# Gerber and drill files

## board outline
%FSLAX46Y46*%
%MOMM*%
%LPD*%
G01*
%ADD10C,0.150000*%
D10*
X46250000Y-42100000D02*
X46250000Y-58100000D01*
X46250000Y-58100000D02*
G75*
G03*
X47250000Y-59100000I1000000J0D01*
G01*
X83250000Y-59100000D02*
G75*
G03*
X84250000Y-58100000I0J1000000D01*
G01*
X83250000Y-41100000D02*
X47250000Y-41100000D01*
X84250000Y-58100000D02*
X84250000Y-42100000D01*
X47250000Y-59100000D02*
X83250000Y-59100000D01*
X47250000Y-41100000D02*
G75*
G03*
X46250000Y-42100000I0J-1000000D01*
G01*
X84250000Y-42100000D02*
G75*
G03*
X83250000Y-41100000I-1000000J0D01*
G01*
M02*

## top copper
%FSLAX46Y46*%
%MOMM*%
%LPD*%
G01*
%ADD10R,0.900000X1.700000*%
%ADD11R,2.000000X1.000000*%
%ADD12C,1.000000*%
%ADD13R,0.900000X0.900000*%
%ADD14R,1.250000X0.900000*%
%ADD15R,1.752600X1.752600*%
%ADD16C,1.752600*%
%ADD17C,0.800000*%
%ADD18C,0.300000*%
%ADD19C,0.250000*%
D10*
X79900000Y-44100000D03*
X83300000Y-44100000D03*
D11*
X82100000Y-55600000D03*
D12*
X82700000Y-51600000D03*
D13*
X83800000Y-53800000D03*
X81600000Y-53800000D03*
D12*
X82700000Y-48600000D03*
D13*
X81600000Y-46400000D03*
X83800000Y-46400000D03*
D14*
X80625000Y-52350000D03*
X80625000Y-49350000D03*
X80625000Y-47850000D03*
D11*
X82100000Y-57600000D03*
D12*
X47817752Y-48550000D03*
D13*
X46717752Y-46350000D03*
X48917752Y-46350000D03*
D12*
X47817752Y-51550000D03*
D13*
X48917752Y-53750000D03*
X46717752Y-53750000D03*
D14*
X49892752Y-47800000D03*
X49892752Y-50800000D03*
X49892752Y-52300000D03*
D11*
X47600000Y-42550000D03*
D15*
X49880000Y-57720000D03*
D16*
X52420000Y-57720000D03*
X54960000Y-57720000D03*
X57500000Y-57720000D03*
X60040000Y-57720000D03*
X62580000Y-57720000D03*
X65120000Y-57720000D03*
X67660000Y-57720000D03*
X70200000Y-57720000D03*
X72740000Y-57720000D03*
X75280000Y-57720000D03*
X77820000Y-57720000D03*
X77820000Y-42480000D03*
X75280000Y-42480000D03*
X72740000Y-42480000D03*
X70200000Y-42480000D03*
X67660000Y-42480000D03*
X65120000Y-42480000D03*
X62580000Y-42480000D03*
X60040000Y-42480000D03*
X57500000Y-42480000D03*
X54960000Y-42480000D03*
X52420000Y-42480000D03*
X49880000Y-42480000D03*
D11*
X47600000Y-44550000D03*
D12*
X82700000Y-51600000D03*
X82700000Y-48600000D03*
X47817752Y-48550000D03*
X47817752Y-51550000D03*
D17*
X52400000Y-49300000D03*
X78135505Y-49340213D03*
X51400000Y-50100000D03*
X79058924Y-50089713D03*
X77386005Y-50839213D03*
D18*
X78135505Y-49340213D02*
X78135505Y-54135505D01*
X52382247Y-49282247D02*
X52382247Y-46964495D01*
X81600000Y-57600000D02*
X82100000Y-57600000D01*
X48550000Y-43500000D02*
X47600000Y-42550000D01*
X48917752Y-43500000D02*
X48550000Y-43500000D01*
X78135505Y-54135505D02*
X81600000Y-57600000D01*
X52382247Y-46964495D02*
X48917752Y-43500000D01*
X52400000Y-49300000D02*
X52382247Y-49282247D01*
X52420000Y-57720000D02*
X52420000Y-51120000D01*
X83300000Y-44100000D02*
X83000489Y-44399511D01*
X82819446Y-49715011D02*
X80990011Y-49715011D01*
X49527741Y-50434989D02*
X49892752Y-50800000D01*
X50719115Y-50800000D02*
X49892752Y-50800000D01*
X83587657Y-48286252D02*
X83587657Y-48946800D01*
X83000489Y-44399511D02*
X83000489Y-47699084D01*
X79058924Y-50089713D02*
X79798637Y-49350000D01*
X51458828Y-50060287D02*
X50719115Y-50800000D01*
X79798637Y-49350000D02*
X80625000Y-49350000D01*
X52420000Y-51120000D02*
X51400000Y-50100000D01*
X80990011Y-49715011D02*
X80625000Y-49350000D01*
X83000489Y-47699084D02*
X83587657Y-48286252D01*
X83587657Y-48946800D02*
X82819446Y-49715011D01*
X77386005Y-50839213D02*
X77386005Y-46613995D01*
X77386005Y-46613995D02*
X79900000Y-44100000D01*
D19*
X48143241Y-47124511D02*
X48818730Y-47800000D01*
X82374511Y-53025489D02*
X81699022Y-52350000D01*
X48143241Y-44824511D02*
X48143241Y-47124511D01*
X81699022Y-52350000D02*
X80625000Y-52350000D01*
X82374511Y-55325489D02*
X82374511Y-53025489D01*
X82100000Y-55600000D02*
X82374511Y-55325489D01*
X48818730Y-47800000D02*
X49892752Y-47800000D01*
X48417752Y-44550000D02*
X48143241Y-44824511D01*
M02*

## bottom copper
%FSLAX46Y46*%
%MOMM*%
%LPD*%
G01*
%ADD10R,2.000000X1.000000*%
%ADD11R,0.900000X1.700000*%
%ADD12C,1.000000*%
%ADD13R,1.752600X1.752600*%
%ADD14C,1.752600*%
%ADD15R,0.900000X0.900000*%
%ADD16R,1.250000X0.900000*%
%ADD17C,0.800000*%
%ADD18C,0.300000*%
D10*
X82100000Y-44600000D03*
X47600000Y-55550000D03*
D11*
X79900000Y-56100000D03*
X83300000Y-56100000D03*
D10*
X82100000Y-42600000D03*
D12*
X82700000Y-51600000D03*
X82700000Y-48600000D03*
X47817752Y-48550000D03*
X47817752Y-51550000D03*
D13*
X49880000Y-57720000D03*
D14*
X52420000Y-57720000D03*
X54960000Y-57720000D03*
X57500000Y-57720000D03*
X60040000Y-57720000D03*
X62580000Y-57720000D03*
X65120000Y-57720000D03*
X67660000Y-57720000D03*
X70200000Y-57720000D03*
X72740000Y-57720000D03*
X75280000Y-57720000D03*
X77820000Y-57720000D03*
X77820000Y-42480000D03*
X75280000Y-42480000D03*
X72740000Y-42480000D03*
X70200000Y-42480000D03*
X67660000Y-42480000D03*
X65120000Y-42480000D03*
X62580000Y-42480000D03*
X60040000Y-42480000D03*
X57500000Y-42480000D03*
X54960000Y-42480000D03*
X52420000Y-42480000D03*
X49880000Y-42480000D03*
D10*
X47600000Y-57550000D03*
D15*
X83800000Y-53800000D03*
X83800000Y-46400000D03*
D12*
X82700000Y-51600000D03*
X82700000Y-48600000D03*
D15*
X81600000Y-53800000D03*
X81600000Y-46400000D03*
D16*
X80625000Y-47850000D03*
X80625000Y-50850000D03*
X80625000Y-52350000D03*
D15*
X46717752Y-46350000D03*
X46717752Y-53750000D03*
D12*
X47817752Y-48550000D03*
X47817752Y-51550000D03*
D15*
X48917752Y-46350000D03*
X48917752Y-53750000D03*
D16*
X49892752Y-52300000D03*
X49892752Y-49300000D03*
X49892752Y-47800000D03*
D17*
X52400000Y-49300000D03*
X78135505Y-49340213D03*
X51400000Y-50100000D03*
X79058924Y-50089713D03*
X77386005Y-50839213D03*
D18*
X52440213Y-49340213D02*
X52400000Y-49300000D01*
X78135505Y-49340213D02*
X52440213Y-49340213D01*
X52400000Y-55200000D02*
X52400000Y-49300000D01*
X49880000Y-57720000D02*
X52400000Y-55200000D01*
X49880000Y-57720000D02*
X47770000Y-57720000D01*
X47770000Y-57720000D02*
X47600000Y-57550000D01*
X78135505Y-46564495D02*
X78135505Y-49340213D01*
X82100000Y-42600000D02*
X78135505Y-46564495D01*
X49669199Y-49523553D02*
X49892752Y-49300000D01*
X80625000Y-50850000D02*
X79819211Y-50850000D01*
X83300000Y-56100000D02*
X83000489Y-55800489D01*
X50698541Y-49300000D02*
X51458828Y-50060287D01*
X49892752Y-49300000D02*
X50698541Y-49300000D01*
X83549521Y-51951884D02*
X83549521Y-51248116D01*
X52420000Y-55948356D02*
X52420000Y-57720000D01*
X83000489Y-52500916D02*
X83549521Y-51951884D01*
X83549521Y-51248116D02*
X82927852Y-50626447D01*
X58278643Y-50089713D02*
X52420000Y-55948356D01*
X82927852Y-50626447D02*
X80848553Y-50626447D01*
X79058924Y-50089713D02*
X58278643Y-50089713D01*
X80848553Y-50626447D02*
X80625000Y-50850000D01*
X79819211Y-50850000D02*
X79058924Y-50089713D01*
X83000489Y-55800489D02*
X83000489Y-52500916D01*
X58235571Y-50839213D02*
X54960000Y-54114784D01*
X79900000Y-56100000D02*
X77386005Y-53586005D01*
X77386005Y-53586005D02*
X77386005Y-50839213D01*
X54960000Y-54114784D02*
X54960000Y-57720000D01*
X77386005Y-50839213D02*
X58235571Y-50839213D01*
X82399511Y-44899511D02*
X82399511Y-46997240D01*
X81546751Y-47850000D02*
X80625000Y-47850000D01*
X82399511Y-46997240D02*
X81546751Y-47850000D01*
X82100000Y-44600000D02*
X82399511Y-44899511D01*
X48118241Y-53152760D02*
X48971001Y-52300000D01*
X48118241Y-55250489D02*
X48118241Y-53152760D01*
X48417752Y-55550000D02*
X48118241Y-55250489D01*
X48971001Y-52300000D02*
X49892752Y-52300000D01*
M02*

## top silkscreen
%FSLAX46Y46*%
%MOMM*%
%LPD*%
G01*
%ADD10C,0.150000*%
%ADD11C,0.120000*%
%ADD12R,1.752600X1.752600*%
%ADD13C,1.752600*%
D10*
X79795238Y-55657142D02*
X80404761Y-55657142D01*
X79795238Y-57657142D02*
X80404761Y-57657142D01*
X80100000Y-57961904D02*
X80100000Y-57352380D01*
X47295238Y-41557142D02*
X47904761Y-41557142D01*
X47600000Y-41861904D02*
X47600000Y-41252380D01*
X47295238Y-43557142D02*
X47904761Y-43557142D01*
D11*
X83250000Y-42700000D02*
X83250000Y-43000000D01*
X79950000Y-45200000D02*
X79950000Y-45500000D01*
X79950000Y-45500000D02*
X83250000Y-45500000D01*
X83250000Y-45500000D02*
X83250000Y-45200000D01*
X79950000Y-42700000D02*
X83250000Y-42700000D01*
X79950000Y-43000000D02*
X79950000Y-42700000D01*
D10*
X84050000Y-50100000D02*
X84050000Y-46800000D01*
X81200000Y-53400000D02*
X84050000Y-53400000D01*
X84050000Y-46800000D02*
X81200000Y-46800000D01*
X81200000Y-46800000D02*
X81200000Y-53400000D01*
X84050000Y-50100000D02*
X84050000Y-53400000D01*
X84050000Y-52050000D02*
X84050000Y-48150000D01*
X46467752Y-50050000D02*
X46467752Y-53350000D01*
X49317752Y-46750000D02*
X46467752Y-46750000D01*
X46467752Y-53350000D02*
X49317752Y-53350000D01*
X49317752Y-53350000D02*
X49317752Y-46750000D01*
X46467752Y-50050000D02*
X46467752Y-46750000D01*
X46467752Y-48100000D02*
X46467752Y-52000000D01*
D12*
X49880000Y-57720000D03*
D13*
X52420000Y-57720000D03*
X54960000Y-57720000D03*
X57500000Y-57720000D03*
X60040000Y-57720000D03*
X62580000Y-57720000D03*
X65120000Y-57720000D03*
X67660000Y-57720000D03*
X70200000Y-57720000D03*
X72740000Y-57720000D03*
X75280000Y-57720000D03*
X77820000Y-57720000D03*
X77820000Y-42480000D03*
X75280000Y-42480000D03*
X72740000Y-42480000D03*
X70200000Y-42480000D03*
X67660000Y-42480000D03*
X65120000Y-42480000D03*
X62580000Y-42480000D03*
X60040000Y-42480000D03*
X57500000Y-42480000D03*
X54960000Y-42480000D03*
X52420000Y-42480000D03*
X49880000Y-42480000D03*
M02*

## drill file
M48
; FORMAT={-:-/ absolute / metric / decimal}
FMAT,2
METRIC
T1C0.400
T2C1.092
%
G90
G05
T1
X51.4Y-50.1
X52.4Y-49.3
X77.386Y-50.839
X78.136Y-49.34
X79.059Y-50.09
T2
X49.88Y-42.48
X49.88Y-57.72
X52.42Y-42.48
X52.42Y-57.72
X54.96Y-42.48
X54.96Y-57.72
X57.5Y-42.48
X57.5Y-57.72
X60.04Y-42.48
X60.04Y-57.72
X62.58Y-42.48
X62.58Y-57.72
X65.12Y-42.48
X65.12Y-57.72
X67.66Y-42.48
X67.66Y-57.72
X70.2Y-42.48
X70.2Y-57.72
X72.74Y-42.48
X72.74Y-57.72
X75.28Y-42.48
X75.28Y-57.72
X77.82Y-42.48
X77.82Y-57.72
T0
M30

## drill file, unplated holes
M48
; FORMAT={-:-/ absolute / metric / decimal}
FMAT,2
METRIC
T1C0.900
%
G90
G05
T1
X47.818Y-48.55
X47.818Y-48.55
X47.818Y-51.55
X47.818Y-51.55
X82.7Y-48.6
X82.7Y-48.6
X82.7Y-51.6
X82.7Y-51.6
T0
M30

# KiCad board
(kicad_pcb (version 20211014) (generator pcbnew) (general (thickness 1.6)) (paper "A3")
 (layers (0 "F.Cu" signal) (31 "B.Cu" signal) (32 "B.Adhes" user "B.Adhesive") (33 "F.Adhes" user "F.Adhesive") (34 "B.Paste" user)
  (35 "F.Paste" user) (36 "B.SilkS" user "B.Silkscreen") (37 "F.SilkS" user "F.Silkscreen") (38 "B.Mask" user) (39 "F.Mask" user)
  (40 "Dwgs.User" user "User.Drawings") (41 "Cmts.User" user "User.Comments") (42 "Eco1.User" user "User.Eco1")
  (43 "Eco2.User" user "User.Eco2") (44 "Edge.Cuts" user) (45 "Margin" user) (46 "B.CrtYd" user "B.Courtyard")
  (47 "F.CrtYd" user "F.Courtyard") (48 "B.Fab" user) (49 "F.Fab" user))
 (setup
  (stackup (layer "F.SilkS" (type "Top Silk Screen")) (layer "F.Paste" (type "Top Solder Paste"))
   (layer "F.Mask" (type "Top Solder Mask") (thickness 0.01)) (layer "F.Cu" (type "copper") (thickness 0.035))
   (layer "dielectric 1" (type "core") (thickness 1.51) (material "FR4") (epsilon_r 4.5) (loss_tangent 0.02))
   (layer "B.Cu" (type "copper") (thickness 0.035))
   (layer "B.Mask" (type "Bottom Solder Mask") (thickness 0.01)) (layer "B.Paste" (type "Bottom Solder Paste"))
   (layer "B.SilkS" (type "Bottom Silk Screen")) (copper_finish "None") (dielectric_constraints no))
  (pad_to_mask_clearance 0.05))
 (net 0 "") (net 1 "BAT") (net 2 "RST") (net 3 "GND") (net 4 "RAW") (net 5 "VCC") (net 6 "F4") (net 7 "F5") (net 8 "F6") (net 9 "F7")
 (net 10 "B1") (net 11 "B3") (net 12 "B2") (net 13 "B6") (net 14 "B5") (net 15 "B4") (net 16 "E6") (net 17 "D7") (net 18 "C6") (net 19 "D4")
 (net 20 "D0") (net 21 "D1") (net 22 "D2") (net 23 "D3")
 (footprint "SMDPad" (layer "F.Cu") (at 82.1 44.6)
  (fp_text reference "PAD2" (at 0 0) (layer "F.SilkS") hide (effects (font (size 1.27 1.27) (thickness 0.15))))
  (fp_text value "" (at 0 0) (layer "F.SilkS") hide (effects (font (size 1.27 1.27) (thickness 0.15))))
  (pad "1" smd rect locked (at 0 0) (size 2 1) (layers "B.Cu" "B.Paste" "B.Mask") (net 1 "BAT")))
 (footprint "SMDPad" (layer "F.Cu") (at 47.6 55.55 180)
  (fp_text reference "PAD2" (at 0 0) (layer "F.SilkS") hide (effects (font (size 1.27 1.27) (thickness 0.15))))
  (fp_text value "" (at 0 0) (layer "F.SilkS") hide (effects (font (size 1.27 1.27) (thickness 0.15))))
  (pad "1" smd rect locked (at 0 0 180) (size 2 1) (layers "B.Cu" "B.Paste" "B.Mask") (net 1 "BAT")))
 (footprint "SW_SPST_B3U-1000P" (layer "F.Cu") (at 81.6 44.1)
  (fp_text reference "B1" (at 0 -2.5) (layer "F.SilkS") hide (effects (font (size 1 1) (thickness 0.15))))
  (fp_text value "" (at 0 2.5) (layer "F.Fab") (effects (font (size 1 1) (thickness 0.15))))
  (fp_line (start 1.65 -1.4) (end 1.65 -1.1) (layer "F.SilkS") (width 0.12))
  (fp_line (start -1.65 1.1) (end -1.65 1.4) (layer "F.SilkS") (width 0.12))
  (fp_line (start -1.65 1.4) (end 1.65 1.4) (layer "F.SilkS") (width 0.12))
  (fp_line (start 1.65 1.4) (end 1.65 1.1) (layer "F.SilkS") (width 0.12))
  (fp_line (start -1.65 -1.4) (end 1.65 -1.4) (layer "F.SilkS") (width 0.12))
  (fp_line (start -1.65 -1.1) (end -1.65 -1.4) (layer "F.SilkS") (width 0.12))
  (pad "1" smd rect locked (at -1.7 0) (size 0.9 1.7) (layers "F.Cu" "F.Paste" "F.Mask") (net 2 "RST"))
  (pad "2" smd rect locked (at 1.7 0) (size 0.9 1.7) (layers "F.Cu" "F.Paste" "F.Mask") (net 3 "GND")))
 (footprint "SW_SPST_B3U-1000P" (layer "F.Cu") (at 81.6 56.1)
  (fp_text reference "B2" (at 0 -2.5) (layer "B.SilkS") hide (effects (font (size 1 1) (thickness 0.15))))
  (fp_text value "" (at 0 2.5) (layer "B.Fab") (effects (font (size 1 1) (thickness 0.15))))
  (pad "1" smd rect locked (at -1.7 0) (size 0.9 1.7) (layers "B.Cu" "B.Paste" "B.Mask") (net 2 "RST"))
  (pad "2" smd rect locked (at 1.7 0) (size 0.9 1.7) (layers "B.Cu" "B.Paste" "B.Mask") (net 3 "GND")))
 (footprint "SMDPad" (layer "F.Cu") (at 82.1 55.6)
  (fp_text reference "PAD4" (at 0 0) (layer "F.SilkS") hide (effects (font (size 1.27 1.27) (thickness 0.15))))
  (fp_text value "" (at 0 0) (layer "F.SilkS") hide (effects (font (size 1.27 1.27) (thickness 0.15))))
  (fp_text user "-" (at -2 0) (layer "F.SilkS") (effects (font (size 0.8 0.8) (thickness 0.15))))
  (pad "1" smd rect locked (at 0 0) (size 2 1) (layers "F.Cu" "F.Paste" "F.Mask") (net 1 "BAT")))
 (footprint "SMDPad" (layer "F.Cu") (at 82.1 42.6)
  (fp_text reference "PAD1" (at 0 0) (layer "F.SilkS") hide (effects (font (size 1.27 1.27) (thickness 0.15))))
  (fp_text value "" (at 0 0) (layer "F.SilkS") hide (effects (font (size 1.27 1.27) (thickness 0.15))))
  (pad "1" smd rect locked (at 0 0) (size 2 1) (layers "B.Cu" "B.Paste" "B.Mask") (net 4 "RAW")))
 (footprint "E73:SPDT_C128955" (layer "F.Cu") (at 82.7 50.1 -90)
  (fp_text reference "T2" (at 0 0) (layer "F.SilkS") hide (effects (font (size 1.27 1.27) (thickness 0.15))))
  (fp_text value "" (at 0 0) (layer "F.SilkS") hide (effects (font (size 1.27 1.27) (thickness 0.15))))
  (fp_line (start 0 -1.35) (end -3.3 -1.35) (layer "F.SilkS") (width 0.15))
  (fp_line (start 3.3 1.5) (end 3.3 -1.35) (layer "F.SilkS") (width 0.15))
  (fp_line (start -3.3 -1.35) (end -3.3 1.5) (layer "F.SilkS") (width 0.15))
  (fp_line (start -3.3 1.5) (end 3.3 1.5) (layer "F.SilkS") (width 0.15))
  (fp_line (start 0 -1.35) (end 3.3 -1.35) (layer "F.SilkS") (width 0.15))
  (fp_line (start 1.95 -1.35) (end -1.95 -1.35) (layer "F.SilkS") (width 0.15))
  (pad "" np_thru_hole circle locked (at 1.5 0) (size 1 1) (drill 0.9) (layers *.Cu *.Mask))
  (pad "" smd rect locked (at 3.7 -1.1 270) (size 0.9 0.9) (layers "F.Cu" "F.Paste" "F.Mask"))
  (pad "" smd rect locked (at 3.7 1.1 270) (size 0.9 0.9) (layers "F.Cu" "F.Paste" "F.Mask"))
  (pad "" np_thru_hole circle locked (at -1.5 0) (size 1 1) (drill 0.9) (layers *.Cu *.Mask))
  (pad "" smd rect locked (at -3.7 1.1 270) (size 0.9 0.9) (layers "F.Cu" "F.Paste" "F.Mask"))
  (pad "" smd rect locked (at -3.7 -1.1 270) (size 0.9 0.9) (layers "F.Cu" "F.Paste" "F.Mask"))
  (pad "1" smd rect locked (at 2.25 2.075 270) (size 0.9 1.25) (layers "F.Cu" "F.Paste" "F.Mask") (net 1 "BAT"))
  (pad "2" smd rect locked (at -0.75 2.075 270) (size 0.9 1.25) (layers "F.Cu" "F.Paste" "F.Mask") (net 3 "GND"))
  (pad "3" smd rect locked (at -2.25 2.075 270) (size 0.9 1.25) (layers "F.Cu" "F.Paste" "F.Mask")))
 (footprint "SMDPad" (layer "F.Cu") (at 82.1 57.6)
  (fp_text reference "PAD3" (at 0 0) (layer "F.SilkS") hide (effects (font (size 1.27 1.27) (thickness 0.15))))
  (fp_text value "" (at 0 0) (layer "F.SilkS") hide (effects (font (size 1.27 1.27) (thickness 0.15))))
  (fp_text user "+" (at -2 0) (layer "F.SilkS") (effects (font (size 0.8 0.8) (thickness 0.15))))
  (pad "1" smd rect locked (at 0 0) (size 2 1) (layers "F.Cu" "F.Paste" "F.Mask") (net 4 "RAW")))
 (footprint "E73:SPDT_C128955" (layer "F.Cu") (at 47.817752 50.05 90)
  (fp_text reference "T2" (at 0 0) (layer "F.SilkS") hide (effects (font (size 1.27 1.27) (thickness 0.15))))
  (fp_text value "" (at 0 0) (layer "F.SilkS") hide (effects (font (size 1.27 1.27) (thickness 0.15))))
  (fp_line (start -3.3 -1.35) (end -3.3 1.5) (layer "F.SilkS") (width 0.15))
  (fp_line (start 3.3 1.5) (end 3.3 -1.35) (layer "F.SilkS") (width 0.15))
  (fp_line (start 0 -1.35) (end 3.3 -1.35) (layer "F.SilkS") (width 0.15))
  (fp_line (start 0 -1.35) (end -3.3 -1.35) (layer "F.SilkS") (width 0.15))
  (fp_line (start 1.95 -1.35) (end -1.95 -1.35) (layer "F.SilkS") (width 0.15))
  (fp_line (start -3.3 1.5) (end 3.3 1.5) (layer "F.SilkS") (width 0.15))
  (pad "" smd rect locked (at -3.7 -1.1 90) (size 0.9 0.9) (layers "F.Cu" "F.Paste" "F.Mask"))
  (pad "" smd rect locked (at -3.7 1.1 90) (size 0.9 0.9) (layers "F.Cu" "F.Paste" "F.Mask"))
  (pad "" np_thru_hole circle locked (at 1.5 0 180) (size 1 1) (drill 0.9) (layers *.Cu *.Mask))
  (pad "" smd rect locked (at 3.7 1.1 90) (size 0.9 0.9) (layers "F.Cu" "F.Paste" "F.Mask"))
  (pad "" smd rect locked (at 3.7 -1.1 90) (size 0.9 0.9) (layers "F.Cu" "F.Paste" "F.Mask"))
  (pad "" np_thru_hole circle locked (at -1.5 0 180) (size 1 1) (drill 0.9) (layers *.Cu *.Mask))
  (pad "1" smd rect locked (at 2.25 2.075 90) (size 0.9 1.25) (layers "F.Cu" "F.Paste" "F.Mask") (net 1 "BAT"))
  (pad "2" smd rect locked (at -0.75 2.075 90) (size 0.9 1.25) (layers "F.Cu" "F.Paste" "F.Mask") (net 3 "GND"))
  (pad "3" smd rect locked (at -2.25 2.075 90) (size 0.9 1.25) (layers "F.Cu" "F.Paste" "F.Mask")))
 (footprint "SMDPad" (layer "F.Cu") (at 47.6 42.55 180)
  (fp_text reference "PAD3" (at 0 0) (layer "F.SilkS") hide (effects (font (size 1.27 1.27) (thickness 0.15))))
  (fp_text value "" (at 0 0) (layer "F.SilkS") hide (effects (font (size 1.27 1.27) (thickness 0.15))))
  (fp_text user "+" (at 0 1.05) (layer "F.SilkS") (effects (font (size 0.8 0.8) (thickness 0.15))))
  (pad "1" smd rect locked (at 0 0 180) (size 2 1) (layers "F.Cu" "F.Paste" "F.Mask") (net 4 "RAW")))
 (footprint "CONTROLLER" (layer "F.Cu") (at 63.85 50.1)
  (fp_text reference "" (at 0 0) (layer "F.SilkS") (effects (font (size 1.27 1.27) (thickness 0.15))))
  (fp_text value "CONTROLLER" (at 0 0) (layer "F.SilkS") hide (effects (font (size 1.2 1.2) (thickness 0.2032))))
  (pad "1" thru_hole rect locked (at -13.97 7.62) (size 1.7526 1.7526) (drill 1.0922) (layers *.Cu *.SilkS *.Mask) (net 4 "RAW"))
  (pad "2" thru_hole circle locked (at -11.43 7.62) (size 1.7526 1.7526) (drill 1.0922) (layers *.Cu *.SilkS *.Mask) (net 3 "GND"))
  (pad "3" thru_hole circle locked (at -8.89 7.62) (size 1.7526 1.7526) (drill 1.0922) (layers *.Cu *.SilkS *.Mask) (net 2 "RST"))
  (pad "4" thru_hole circle locked (at -6.35 7.62) (size 1.7526 1.7526) (drill 1.0922) (layers *.Cu *.SilkS *.Mask) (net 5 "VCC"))
  (pad "5" thru_hole circle locked (at -3.81 7.62) (size 1.7526 1.7526) (drill 1.0922) (layers *.Cu *.SilkS *.Mask) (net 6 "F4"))
  (pad "6" thru_hole circle locked (at -1.27 7.62) (size 1.7526 1.7526) (drill 1.0922) (layers *.Cu *.SilkS *.Mask) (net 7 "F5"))
  (pad "7" thru_hole circle locked (at 1.27 7.62) (size 1.7526 1.7526) (drill 1.0922) (layers *.Cu *.SilkS *.Mask) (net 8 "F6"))
  (pad "8" thru_hole circle locked (at 3.81 7.62) (size 1.7526 1.7526) (drill 1.0922) (layers *.Cu *.SilkS *.Mask) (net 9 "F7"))
  (pad "9" thru_hole circle locked (at 6.35 7.62) (size 1.7526 1.7526) (drill 1.0922) (layers *.Cu *.SilkS *.Mask) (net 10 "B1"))
  (pad "10" thru_hole circle locked (at 8.89 7.62) (size 1.7526 1.7526) (drill 1.0922) (layers *.Cu *.SilkS *.Mask) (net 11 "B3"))
  (pad "11" thru_hole circle locked (at 11.43 7.62) (size 1.7526 1.7526) (drill 1.0922) (layers *.Cu *.SilkS *.Mask) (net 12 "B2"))
  (pad "12" thru_hole circle locked (at 13.97 7.62) (size 1.7526 1.7526) (drill 1.0922) (layers *.Cu *.SilkS *.Mask) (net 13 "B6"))
  (pad "13" thru_hole circle locked (at 13.97 -7.62) (size 1.7526 1.7526) (drill 1.0922) (layers *.Cu *.SilkS *.Mask) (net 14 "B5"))
  (pad "14" thru_hole circle locked (at 11.43 -7.62) (size 1.7526 1.7526) (drill 1.0922) (layers *.Cu *.SilkS *.Mask) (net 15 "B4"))
  (pad "15" thru_hole circle locked (at 8.89 -7.62) (size 1.7526 1.7526) (drill 1.0922) (layers *.Cu *.SilkS *.Mask) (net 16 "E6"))
  (pad "16" thru_hole circle locked (at 6.35 -7.62) (size 1.7526 1.7526) (drill 1.0922) (layers *.Cu *.SilkS *.Mask) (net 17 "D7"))
  (pad "17" thru_hole circle locked (at 3.81 -7.62) (size 1.7526 1.7526) (drill 1.0922) (layers *.Cu *.SilkS *.Mask) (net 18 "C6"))
  (pad "18" thru_hole circle locked (at 1.27 -7.62) (size 1.7526 1.7526) (drill 1.0922) (layers *.Cu *.SilkS *.Mask) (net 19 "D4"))
  (pad "19" thru_hole circle locked (at -1.27 -7.62) (size 1.7526 1.7526) (drill 1.0922) (layers *.Cu *.SilkS *.Mask) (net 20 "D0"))
  (pad "20" thru_hole circle locked (at -3.81 -7.62) (size 1.7526 1.7526) (drill 1.0922) (layers *.Cu *.SilkS *.Mask) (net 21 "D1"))
  (pad "21" thru_hole circle locked (at -6.35 -7.62) (size 1.7526 1.7526) (drill 1.0922) (layers *.Cu *.SilkS *.Mask) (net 3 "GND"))
  (pad "22" thru_hole circle locked (at -8.89 -7.62) (size 1.7526 1.7526) (drill 1.0922) (layers *.Cu *.SilkS *.Mask) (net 3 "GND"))
  (pad "23" thru_hole circle locked (at -11.43 -7.62) (size 1.7526 1.7526) (drill 1.0922) (layers *.Cu *.SilkS *.Mask) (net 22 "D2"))
  (pad "24" thru_hole circle locked (at -13.97 -7.62) (size 1.7526 1.7526) (drill 1.0922) (layers *.Cu *.SilkS *.Mask) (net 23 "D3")))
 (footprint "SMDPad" (layer "F.Cu") (at 47.6 44.55 180)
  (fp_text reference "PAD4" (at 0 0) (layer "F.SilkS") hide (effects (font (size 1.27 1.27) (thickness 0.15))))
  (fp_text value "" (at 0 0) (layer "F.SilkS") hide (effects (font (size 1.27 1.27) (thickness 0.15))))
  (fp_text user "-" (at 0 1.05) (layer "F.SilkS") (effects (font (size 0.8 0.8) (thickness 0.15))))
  (pad "1" smd rect locked (at 0 0 180) (size 2 1) (layers "F.Cu" "F.Paste" "F.Mask") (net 1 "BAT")))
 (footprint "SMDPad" (layer "F.Cu") (at 47.6 57.55 180)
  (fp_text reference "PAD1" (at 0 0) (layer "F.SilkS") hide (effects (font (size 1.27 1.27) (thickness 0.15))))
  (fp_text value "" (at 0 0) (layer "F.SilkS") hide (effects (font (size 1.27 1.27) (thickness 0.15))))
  (pad "1" smd rect locked (at 0 0 180) (size 2 1) (layers "B.Cu" "B.Paste" "B.Mask") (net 4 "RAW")))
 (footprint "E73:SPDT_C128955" (layer "B.Cu") (at 82.7 50.1 -90)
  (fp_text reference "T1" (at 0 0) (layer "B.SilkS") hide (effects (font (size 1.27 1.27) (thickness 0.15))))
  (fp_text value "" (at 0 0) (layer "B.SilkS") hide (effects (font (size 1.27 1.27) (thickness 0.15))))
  (pad "" smd rect locked (at 3.7 -1.1 270) (size 0.9 0.9) (layers "B.Cu" "B.Paste" "B.Mask"))
  (pad "" smd rect locked (at -3.7 -1.1 270) (size 0.9 0.9) (layers "B.Cu" "B.Paste" "B.Mask"))
  (pad "" np_thru_hole circle locked (at 1.5 0) (size 1 1) (drill 0.9) (layers *.Cu *.Mask))
  (pad "" np_thru_hole circle locked (at -1.5 0) (size 1 1) (drill 0.9) (layers *.Cu *.Mask))
  (pad "" smd rect locked (at 3.7 1.1 270) (size 0.9 0.9) (layers "B.Cu" "B.Paste" "B.Mask"))
  (pad "" smd rect locked (at -3.7 1.1 270) (size 0.9 0.9) (layers "B.Cu" "B.Paste" "B.Mask"))
  (pad "1" smd rect locked (at -2.25 2.075 270) (size 0.9 1.25) (layers "B.Cu" "B.Paste" "B.Mask") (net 1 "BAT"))
  (pad "2" smd rect locked (at 0.75 2.075 270) (size 0.9 1.25) (layers "B.Cu" "B.Paste" "B.Mask") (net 3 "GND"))
  (pad "3" smd rect locked (at 2.25 2.075 270) (size 0.9 1.25) (layers "B.Cu" "B.Paste" "B.Mask")))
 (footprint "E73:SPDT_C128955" (layer "B.Cu") (at 47.817752 50.05 90)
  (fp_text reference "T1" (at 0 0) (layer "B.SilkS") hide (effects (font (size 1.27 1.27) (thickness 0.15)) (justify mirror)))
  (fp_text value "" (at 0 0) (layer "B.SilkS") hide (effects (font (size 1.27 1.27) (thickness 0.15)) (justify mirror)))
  (pad "" smd rect locked (at 3.7 1.1 90) (size 0.9 0.9) (layers "B.Cu" "B.Paste" "B.Mask"))
  (pad "" smd rect locked (at -3.7 -1.1 90) (size 0.9 0.9) (layers "B.Cu" "B.Paste" "B.Mask"))
  (pad "" np_thru_hole circle locked (at 1.5 0 180) (size 1 1) (drill 0.9) (layers *.Cu *.Mask))
  (pad "" np_thru_hole circle locked (at -1.5 0 180) (size 1 1) (drill 0.9) (layers *.Cu *.Mask))
  (pad "" smd rect locked (at 3.7 -1.1 90) (size 0.9 0.9) (layers "B.Cu" "B.Paste" "B.Mask"))
  (pad "" smd rect locked (at -3.7 1.1 90) (size 0.9 0.9) (layers "B.Cu" "B.Paste" "B.Mask"))
  (pad "1" smd rect locked (at -2.25 2.075 90) (size 0.9 1.25) (layers "B.Cu" "B.Paste" "B.Mask") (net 1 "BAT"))
  (pad "2" smd rect locked (at 0.75 2.075 90) (size 0.9 1.25) (layers "B.Cu" "B.Paste" "B.Mask") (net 3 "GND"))
  (pad "3" smd rect locked (at 2.25 2.075 90) (size 0.9 1.25) (layers "B.Cu" "B.Paste" "B.Mask")))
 (gr_line (start 46.25 42.1) (end 46.25 58.1) (layer "Edge.Cuts") (width 0.15))
 (gr_arc (start 47.25 59.1) (mid 46.542893 58.807107) (end 46.25 58.1) (layer "Edge.Cuts") (width 0.15))
 (gr_arc (start 84.25 58.1) (mid 83.957107 58.807107) (end 83.25 59.1) (layer "Edge.Cuts") (width 0.15))
 (gr_line (start 83.25 41.1) (end 47.25 41.1) (layer "Edge.Cuts") (width 0.15))
 (gr_line (start 84.25 58.1) (end 84.25 42.1) (layer "Edge.Cuts") (width 0.15))
 (gr_line (start 47.25 59.1) (end 83.25 59.1) (layer "Edge.Cuts") (width 0.15))
 (gr_arc (start 46.25 42.1) (mid 46.542893 41.392893) (end 47.25 41.1) (layer "Edge.Cuts") (width 0.15))
 (gr_arc (start 83.25 41.1) (mid 83.957107 41.392893) (end 84.25 42.1) (layer "Edge.Cuts") (width 0.15))
 (segment (start 78.135505 49.340213) (end 78.135505 54.135505) (width 0.3) (layer "F.Cu") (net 4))
 (segment (start 52.382247 49.282247) (end 52.382247 46.964495) (width 0.3) (layer "F.Cu") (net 4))
 (segment (start 81.6 57.6) (end 82.1 57.6) (width 0.3) (layer "F.Cu") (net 4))
 (segment (start 48.55 43.5) (end 47.6 42.55) (width 0.3) (layer "F.Cu") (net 4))
 (segment (start 48.917752 43.5) (end 48.55 43.5) (width 0.3) (layer "F.Cu") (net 4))
 (segment (start 78.135505 54.135505) (end 81.6 57.6) (width 0.3) (layer "F.Cu") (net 4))
 (segment (start 52.382247 46.964495) (end 48.917752 43.5) (width 0.3) (layer "F.Cu") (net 4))
 (segment (start 52.4 49.3) (end 52.382247 49.282247) (width 0.3) (layer "F.Cu") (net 4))
 (via (at 52.4 49.3) (size 0.8) (drill 0.4) (layers "F.Cu" "B.Cu") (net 4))
 (via (at 78.135505 49.340213) (size 0.8) (drill 0.4) (layers "F.Cu" "B.Cu") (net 4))
 (segment (start 49.88 57.72) (end 52.4 55.2) (width 0.3) (layer "B.Cu") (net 4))
 (segment (start 49.88 57.72) (end 47.77 57.72) (width 0.3) (layer "B.Cu") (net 4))
 (segment (start 47.77 57.72) (end 47.6 57.55) (width 0.3) (layer "B.Cu") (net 4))
 (segment (start 52.440213 49.340213) (end 52.4 49.3) (width 0.3) (layer "B.Cu") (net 4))
 (segment (start 78.135505 46.564495) (end 78.135505 49.340213) (width 0.3) (layer "B.Cu") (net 4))
 (segment (start 52.4 55.2) (end 52.4 49.3) (width 0.3) (layer "B.Cu") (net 4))
 (segment (start 78.135505 49.340213) (end 52.440213 49.340213) (width 0.3) (layer "B.Cu") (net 4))
 (segment (start 82.1 42.6) (end 78.135505 46.564495) (width 0.3) (layer "B.Cu") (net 4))
 (segment (start 52.42 57.72) (end 52.42 51.12) (width 0.3) (layer "F.Cu") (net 3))
 (segment (start 83.3 44.1) (end 83.000489 44.399511) (width 0.3) (layer "F.Cu") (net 3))
 (segment (start 82.819446 49.715011) (end 80.990011 49.715011) (width 0.3) (layer "F.Cu") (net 3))
 (segment (start 49.527741 50.434989) (end 49.892752 50.8) (width 0.3) (layer "F.Cu") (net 3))
 (segment (start 50.719115 50.8) (end 49.892752 50.8) (width 0.3) (layer "F.Cu") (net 3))
 (segment (start 83.587657 48.286252) (end 83.587657 48.9468) (width 0.3) (layer "F.Cu") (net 3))
 (segment (start 83.000489 44.399511) (end 83.000489 47.699084) (width 0.3) (layer "F.Cu") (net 3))
 (segment (start 79.058924 50.089713) (end 79.798637 49.35) (width 0.3) (layer "F.Cu") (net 3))
 (segment (start 51.458828 50.060287) (end 50.719115 50.8) (width 0.3) (layer "F.Cu") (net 3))
 (segment (start 79.798637 49.35) (end 80.625 49.35) (width 0.3) (layer "F.Cu") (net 3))
 (segment (start 52.42 51.12) (end 51.4 50.1) (width 0.3) (layer "F.Cu") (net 3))
 (segment (start 80.990011 49.715011) (end 80.625 49.35) (width 0.3) (layer "F.Cu") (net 3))
 (segment (start 83.000489 47.699084) (end 83.587657 48.286252) (width 0.3) (layer "F.Cu") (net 3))
 (segment (start 83.587657 48.9468) (end 82.819446 49.715011) (width 0.3) (layer "F.Cu") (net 3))
 (via (at 51.4 50.1) (size 0.8) (drill 0.4) (layers "F.Cu" "B.Cu") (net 3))
 (via (at 79.058924 50.089713) (size 0.8) (drill 0.4) (layers "F.Cu" "B.Cu") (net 3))
 (segment (start 49.669199 49.523553) (end 49.892752 49.3) (width 0.3) (layer "B.Cu") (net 3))
 (segment (start 80.625 50.85) (end 79.819211 50.85) (width 0.3) (layer "B.Cu") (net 3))
 (segment (start 83.3 56.1) (end 83.000489 55.800489) (width 0.3) (layer "B.Cu") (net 3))
 (segment (start 50.698541 49.3) (end 51.458828 50.060287) (width 0.3) (layer "B.Cu") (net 3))
 (segment (start 49.892752 49.3) (end 50.698541 49.3) (width 0.3) (layer "B.Cu") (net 3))
 (segment (start 83.549521 51.951884) (end 83.549521 51.248116) (width 0.3) (layer "B.Cu") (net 3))
 (segment (start 52.42 55.948356) (end 52.42 57.72) (width 0.3) (layer "B.Cu") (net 3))
 (segment (start 83.000489 52.500916) (end 83.549521 51.951884) (width 0.3) (layer "B.Cu") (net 3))
 (segment (start 83.549521 51.248116) (end 82.927852 50.626447) (width 0.3) (layer "B.Cu") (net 3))
 (segment (start 58.278643 50.089713) (end 52.42 55.948356) (width 0.3) (layer "B.Cu") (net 3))
 (segment (start 82.927852 50.626447) (end 80.848553 50.626447) (width 0.3) (layer "B.Cu") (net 3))
 (segment (start 79.058924 50.089713) (end 58.278643 50.089713) (width 0.3) (layer "B.Cu") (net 3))
 (segment (start 80.848553 50.626447) (end 80.625 50.85) (width 0.3) (layer "B.Cu") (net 3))
 (segment (start 79.819211 50.85) (end 79.058924 50.089713) (width 0.3) (layer "B.Cu") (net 3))
 (segment (start 83.000489 55.800489) (end 83.000489 52.500916) (width 0.3) (layer "B.Cu") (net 3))
 (segment (start 77.386005 50.839213) (end 77.386005 46.613995) (width 0.3) (layer "F.Cu") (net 2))
 (segment (start 77.386005 46.613995) (end 79.9 44.1) (width 0.3) (layer "F.Cu") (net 2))
 (via (at 77.386005 50.839213) (size 0.8) (drill 0.4) (layers "F.Cu" "B.Cu") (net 2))
 (segment (start 58.235571 50.839213) (end 54.96 54.114784) (width 0.3) (layer "B.Cu") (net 2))
 (segment (start 79.9 56.1) (end 77.386005 53.586005) (width 0.3) (layer "B.Cu") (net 2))
 (segment (start 77.386005 53.586005) (end 77.386005 50.839213) (width 0.3) (layer "B.Cu") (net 2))
 (segment (start 54.96 54.114784) (end 54.96 57.72) (width 0.3) (layer "B.Cu") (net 2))
 (segment (start 77.386005 50.839213) (end 58.235571 50.839213) (width 0.3) (layer "B.Cu") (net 2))
 (segment (start 48.143241 47.124511) (end 48.81873 47.8) (width 0.25) (layer "F.Cu") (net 1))
 (segment (start 82.374511 53.025489) (end 81.699022 52.35) (width 0.25) (layer "F.Cu") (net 1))
 (segment (start 48.143241 44.824511) (end 48.143241 47.124511) (width 0.25) (layer "F.Cu") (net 1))
 (segment (start 81.699022 52.35) (end 80.625 52.35) (width 0.25) (layer "F.Cu") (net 1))
 (segment (start 82.374511 55.325489) (end 82.374511 53.025489) (width 0.25) (layer "F.Cu") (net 1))
 (segment (start 82.1 55.6) (end 82.374511 55.325489) (width 0.25) (layer "F.Cu") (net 1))
 (segment (start 48.81873 47.8) (end 49.892752 47.8) (width 0.25) (layer "F.Cu") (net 1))
 (segment (start 48.417752 44.55) (end 48.143241 44.824511) (width 0.25) (layer "F.Cu") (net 1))
 (segment (start 82.399511 44.899511) (end 82.399511 46.99724) (width 0.3) (layer "B.Cu") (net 1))
 (segment (start 81.546751 47.85) (end 80.625 47.85) (width 0.3) (layer "B.Cu") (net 1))
 (segment (start 82.399511 46.99724) (end 81.546751 47.85) (width 0.3) (layer "B.Cu") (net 1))
 (segment (start 82.1 44.6) (end 82.399511 44.899511) (width 0.3) (layer "B.Cu") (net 1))
 (segment (start 48.118241 53.15276) (end 48.971001 52.3) (width 0.3) (layer "B.Cu") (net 1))
 (segment (start 48.118241 55.250489) (end 48.118241 53.15276) (width 0.3) (layer "B.Cu") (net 1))
 (segment (start 48.417752 55.55) (end 48.118241 55.250489) (width 0.3) (layer "B.Cu") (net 1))
 (segment (start 48.971001 52.3) (end 49.892752 52.3) (width 0.3) (layer "B.Cu") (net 1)))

